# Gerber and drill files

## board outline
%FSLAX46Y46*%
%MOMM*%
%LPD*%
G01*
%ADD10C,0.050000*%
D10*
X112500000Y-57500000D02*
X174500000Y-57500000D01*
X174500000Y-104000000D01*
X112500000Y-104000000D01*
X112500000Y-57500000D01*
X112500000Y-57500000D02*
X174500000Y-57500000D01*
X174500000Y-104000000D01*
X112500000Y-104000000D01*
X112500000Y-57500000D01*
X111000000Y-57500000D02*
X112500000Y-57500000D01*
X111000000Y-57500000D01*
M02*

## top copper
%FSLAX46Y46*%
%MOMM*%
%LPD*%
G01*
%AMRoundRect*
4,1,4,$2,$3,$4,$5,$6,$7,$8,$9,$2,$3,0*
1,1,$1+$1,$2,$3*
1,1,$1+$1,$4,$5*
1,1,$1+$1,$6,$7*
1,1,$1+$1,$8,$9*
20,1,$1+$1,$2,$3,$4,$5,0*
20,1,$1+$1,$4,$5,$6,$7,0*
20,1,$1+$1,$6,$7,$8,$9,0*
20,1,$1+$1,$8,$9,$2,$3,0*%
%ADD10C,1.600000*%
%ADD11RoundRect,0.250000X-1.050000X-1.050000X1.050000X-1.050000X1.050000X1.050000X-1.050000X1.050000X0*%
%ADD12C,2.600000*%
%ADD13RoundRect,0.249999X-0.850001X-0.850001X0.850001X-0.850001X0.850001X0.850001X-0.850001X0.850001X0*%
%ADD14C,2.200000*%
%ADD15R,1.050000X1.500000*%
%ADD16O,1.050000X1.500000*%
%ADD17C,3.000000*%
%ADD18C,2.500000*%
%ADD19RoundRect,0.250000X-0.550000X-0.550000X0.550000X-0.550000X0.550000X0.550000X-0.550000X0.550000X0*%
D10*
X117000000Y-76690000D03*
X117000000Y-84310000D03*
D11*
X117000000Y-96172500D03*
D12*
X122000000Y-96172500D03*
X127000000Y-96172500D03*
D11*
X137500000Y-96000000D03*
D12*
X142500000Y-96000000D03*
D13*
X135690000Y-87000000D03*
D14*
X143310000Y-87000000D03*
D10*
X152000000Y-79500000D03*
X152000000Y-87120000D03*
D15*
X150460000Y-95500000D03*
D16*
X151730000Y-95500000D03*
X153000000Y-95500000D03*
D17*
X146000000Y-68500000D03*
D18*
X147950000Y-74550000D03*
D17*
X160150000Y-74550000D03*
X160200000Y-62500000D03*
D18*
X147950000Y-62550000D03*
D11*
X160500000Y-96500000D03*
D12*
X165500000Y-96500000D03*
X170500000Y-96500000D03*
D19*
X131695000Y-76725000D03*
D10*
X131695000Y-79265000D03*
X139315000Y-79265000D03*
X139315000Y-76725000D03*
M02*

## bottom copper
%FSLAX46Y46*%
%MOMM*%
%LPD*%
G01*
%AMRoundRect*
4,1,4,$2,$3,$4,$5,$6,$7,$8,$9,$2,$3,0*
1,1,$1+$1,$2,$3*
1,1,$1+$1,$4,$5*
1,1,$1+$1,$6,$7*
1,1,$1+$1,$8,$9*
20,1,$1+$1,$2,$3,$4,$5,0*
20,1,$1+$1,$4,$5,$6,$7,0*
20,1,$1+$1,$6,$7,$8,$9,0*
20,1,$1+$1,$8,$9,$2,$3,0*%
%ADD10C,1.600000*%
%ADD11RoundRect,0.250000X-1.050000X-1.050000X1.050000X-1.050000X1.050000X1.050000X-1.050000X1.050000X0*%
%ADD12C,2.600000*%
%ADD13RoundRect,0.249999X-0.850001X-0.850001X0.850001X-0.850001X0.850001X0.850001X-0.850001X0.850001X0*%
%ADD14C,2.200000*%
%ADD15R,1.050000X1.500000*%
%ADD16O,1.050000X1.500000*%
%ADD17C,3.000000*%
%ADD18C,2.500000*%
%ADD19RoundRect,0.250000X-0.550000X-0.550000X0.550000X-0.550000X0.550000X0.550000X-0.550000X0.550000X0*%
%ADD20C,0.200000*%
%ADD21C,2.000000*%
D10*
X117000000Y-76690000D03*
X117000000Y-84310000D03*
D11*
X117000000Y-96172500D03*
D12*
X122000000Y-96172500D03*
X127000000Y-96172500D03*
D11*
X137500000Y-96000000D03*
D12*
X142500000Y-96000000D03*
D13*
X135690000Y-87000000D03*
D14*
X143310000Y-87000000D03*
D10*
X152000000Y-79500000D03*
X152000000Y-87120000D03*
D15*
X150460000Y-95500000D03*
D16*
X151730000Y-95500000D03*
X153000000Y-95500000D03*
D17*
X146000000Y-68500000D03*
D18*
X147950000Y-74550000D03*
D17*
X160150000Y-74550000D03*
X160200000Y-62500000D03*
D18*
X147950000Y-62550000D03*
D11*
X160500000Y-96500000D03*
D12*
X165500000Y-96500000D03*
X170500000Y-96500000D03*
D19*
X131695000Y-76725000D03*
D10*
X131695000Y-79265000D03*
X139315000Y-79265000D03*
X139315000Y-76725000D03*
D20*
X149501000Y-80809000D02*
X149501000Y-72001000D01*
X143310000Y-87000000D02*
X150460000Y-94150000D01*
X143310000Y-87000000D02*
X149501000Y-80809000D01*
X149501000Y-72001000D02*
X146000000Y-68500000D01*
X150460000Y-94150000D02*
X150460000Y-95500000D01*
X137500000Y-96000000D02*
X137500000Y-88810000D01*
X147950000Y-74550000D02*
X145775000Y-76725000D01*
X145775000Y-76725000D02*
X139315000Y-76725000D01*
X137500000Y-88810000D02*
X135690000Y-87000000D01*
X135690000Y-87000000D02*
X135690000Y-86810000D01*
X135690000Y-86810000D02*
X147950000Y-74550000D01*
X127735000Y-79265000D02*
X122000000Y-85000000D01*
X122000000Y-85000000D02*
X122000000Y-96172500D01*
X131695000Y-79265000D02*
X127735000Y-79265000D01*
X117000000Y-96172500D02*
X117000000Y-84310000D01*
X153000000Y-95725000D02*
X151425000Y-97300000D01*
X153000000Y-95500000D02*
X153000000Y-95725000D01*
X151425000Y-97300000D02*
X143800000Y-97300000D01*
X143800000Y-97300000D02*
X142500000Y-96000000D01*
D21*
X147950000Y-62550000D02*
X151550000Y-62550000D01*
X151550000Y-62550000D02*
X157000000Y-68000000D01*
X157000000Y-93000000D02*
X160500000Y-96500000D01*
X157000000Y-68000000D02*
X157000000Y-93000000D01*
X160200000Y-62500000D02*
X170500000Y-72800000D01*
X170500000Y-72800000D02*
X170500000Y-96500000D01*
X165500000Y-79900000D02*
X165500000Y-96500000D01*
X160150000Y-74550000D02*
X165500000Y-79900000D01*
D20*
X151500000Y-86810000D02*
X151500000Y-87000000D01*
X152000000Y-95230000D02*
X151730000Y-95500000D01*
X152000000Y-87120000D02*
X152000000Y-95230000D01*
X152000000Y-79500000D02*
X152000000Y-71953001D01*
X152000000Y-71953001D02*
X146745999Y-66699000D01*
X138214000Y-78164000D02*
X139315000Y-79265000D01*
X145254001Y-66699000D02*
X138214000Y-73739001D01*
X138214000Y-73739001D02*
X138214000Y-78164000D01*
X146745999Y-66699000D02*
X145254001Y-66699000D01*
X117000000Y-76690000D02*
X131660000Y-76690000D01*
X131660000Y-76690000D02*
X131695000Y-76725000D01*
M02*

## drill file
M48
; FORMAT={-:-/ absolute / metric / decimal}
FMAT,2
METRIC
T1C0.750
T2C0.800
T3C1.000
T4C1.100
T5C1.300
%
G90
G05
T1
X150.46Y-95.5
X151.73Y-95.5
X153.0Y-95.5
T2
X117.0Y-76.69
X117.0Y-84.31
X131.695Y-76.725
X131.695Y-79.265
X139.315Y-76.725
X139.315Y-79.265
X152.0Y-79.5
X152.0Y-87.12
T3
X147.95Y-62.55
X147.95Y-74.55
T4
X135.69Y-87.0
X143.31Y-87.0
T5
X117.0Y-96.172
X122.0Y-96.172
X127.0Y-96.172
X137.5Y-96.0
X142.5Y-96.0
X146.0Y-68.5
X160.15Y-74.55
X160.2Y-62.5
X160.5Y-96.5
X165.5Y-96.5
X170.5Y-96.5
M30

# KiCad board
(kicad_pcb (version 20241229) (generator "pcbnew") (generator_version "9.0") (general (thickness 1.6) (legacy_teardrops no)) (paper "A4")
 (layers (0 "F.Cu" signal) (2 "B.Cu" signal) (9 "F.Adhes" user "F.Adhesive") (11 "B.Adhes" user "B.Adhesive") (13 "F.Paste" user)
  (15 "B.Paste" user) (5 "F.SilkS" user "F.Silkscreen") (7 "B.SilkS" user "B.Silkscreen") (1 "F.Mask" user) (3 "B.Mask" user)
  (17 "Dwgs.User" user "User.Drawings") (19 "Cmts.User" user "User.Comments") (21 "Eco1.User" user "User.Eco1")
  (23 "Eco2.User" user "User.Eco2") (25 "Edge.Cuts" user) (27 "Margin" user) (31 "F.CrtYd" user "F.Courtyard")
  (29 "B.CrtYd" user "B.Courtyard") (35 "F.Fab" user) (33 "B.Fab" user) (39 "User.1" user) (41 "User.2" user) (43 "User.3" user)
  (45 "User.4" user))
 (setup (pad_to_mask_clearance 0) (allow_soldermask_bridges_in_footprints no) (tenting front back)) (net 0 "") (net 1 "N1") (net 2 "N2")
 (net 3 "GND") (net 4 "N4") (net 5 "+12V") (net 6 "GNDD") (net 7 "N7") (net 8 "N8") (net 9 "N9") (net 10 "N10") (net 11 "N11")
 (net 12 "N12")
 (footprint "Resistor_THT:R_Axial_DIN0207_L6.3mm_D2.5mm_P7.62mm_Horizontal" (layer "F.Cu") (at 117 76.69 -90)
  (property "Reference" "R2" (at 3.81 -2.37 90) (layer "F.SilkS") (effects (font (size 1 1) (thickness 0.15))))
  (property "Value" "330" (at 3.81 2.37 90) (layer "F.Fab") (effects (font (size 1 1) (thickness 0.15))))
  (pad "1" thru_hole circle (at 0 0 270) (size 1.6 1.6) (drill 0.8) (layers "*.Cu" "*.Mask") (remove_unused_layers no) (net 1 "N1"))
  (pad "2" thru_hole circle (at 7.62 0 270) (size 1.6 1.6) (drill 0.8) (layers "*.Cu" "*.Mask") (remove_unused_layers no) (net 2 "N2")))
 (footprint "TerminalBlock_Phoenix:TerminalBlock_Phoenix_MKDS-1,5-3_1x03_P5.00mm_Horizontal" (layer "F.Cu") (at 117 96.1725)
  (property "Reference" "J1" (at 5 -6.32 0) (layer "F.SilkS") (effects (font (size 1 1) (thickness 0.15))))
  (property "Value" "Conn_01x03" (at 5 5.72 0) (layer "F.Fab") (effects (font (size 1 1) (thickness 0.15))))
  (pad "1" thru_hole roundrect (at 0 0) (size 2.6 2.6) (drill 1.3) (layers "*.Cu" "*.Mask") (remove_unused_layers no)
   (roundrect_rratio 0.096154) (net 2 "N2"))
  (pad "2" thru_hole circle (at 5 0) (size 2.6 2.6) (drill 1.3) (layers "*.Cu" "*.Mask") (remove_unused_layers no) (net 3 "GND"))
  (pad "3" thru_hole circle (at 10 0) (size 2.6 2.6) (drill 1.3) (layers "*.Cu" "*.Mask") (remove_unused_layers no) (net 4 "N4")))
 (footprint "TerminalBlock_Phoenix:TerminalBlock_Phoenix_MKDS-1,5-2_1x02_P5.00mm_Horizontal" (layer "F.Cu") (at 137.5 96)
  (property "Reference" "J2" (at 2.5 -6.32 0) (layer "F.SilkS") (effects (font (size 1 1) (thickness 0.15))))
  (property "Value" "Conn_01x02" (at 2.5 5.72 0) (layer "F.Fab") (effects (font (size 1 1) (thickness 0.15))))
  (pad "1" thru_hole roundrect (at 0 0) (size 2.6 2.6) (drill 1.3) (layers "*.Cu" "*.Mask") (remove_unused_layers no)
   (roundrect_rratio 0.096154) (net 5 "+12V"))
  (pad "2" thru_hole circle (at 5 0) (size 2.6 2.6) (drill 1.3) (layers "*.Cu" "*.Mask") (remove_unused_layers no) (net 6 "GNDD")))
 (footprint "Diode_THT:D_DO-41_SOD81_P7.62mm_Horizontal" (layer "F.Cu") (at 135.69 87)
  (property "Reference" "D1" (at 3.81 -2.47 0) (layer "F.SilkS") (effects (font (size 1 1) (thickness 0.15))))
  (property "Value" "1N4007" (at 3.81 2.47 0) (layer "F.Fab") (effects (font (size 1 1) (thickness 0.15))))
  (pad "1" thru_hole roundrect (at 0 0) (size 2.2 2.2) (drill 1.1) (layers "*.Cu" "*.Mask") (remove_unused_layers no)
   (roundrect_rratio 0.113636) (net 5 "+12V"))
  (pad "2" thru_hole circle (at 7.62 0) (size 2.2 2.2) (drill 1.1) (layers "*.Cu" "*.Mask") (remove_unused_layers no) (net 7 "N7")))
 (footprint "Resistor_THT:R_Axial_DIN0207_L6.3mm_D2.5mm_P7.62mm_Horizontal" (layer "F.Cu") (at 152 79.5 -90)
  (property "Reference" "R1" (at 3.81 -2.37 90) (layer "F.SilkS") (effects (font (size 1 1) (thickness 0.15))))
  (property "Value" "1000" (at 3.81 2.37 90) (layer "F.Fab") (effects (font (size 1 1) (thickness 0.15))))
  (pad "1" thru_hole circle (at 0 0 270) (size 1.6 1.6) (drill 0.8) (layers "*.Cu" "*.Mask") (remove_unused_layers no) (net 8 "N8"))
  (pad "2" thru_hole circle (at 7.62 0 270) (size 1.6 1.6) (drill 0.8) (layers "*.Cu" "*.Mask") (remove_unused_layers no) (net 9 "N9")))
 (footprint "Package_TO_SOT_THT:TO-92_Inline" (layer "F.Cu") (at 150.46 95.5)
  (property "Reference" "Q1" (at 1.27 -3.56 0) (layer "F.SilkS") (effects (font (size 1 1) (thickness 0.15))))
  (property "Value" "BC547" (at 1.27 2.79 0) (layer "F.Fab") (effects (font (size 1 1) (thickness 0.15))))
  (pad "1" thru_hole rect (at 0 0) (size 1.05 1.5) (drill 0.75) (layers "*.Cu" "*.Mask") (remove_unused_layers no) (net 7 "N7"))
  (pad "2" thru_hole oval (at 1.27 0) (size 1.05 1.5) (drill 0.75) (layers "*.Cu" "*.Mask") (remove_unused_layers no) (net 9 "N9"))
  (pad "3" thru_hole oval (at 2.54 0) (size 1.05 1.5) (drill 0.75) (layers "*.Cu" "*.Mask") (remove_unused_layers no) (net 6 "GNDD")))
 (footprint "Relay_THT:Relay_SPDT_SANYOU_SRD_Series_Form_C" (layer "F.Cu") (at 146 68.5)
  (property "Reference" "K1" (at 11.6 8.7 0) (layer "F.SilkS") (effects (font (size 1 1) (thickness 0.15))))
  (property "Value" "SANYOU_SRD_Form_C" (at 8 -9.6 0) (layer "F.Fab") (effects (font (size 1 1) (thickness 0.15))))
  (pad "1" thru_hole circle (at 0 0 90) (size 3 3) (drill 1.3) (layers "*.Cu" "*.Mask") (remove_unused_layers no) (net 7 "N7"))
  (pad "2" thru_hole circle (at 1.95 6.05 90) (size 2.5 2.5) (drill 1) (layers "*.Cu" "*.Mask") (remove_unused_layers no) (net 5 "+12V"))
  (pad "3" thru_hole circle (at 14.15 6.05 90) (size 3 3) (drill 1.3) (layers "*.Cu" "*.Mask") (remove_unused_layers no) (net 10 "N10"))
  (pad "4" thru_hole circle (at 14.2 -6 90) (size 3 3) (drill 1.3) (layers "*.Cu" "*.Mask") (remove_unused_layers no) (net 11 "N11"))
  (pad "5" thru_hole circle (at 1.95 -5.95 90) (size 2.5 2.5) (drill 1) (layers "*.Cu" "*.Mask") (remove_unused_layers no) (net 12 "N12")))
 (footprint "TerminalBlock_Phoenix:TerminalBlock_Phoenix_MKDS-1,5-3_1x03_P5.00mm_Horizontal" (layer "F.Cu") (at 160.5 96.5)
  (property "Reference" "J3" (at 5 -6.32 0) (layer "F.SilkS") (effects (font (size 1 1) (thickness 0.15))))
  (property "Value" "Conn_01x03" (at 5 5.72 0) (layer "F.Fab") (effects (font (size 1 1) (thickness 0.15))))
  (pad "1" thru_hole roundrect (at 0 0) (size 2.6 2.6) (drill 1.3) (layers "*.Cu" "*.Mask") (remove_unused_layers no)
   (roundrect_rratio 0.096154) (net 12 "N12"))
  (pad "2" thru_hole circle (at 5 0) (size 2.6 2.6) (drill 1.3) (layers "*.Cu" "*.Mask") (remove_unused_layers no) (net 10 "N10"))
  (pad "3" thru_hole circle (at 10 0) (size 2.6 2.6) (drill 1.3) (layers "*.Cu" "*.Mask") (remove_unused_layers no) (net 11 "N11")))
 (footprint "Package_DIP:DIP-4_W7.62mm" (layer "F.Cu") (at 131.695 76.725)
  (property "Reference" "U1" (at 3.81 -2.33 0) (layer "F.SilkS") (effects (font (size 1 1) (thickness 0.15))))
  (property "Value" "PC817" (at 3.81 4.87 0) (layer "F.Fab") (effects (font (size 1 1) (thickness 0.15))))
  (pad "1" thru_hole roundrect (at 0 0) (size 1.6 1.6) (drill 0.8) (layers "*.Cu" "*.Mask") (remove_unused_layers no)
   (roundrect_rratio 0.15625) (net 1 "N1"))
  (pad "2" thru_hole circle (at 0 2.54) (size 1.6 1.6) (drill 0.8) (layers "*.Cu" "*.Mask") (remove_unused_layers no) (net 3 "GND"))
  (pad "3" thru_hole circle (at 7.62 2.54) (size 1.6 1.6) (drill 0.8) (layers "*.Cu" "*.Mask") (remove_unused_layers no) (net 8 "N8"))
  (pad "4" thru_hole circle (at 7.62 0) (size 1.6 1.6) (drill 0.8) (layers "*.Cu" "*.Mask") (remove_unused_layers no) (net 5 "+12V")))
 (gr_rect (start 112.5 57.5) (end 174.5 104) (stroke (width 0.05) (type default)) (fill no) (layer "Edge.Cuts"))
 (gr_rect (start 112.5 57.5) (end 174.5 104) (stroke (width 0.05) (type default)) (fill no) (layer "Edge.Cuts"))
 (gr_rect (start 111 57.5) (end 112.5 57.5) (stroke (width 0.05) (type default)) (fill no) (layer "Edge.Cuts"))
 (segment (start 149.501 80.809) (end 149.501 72.001) (width 0.2) (layer "B.Cu") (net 7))
 (segment (start 143.31 87) (end 150.46 94.15) (width 0.2) (layer "B.Cu") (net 7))
 (segment (start 143.31 87) (end 149.501 80.809) (width 0.2) (layer "B.Cu") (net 7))
 (segment (start 149.501 72.001) (end 146 68.5) (width 0.2) (layer "B.Cu") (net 7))
 (segment (start 150.46 94.15) (end 150.46 95.5) (width 0.2) (layer "B.Cu") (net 7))
 (segment (start 137.5 96) (end 137.5 88.81) (width 0.2) (layer "B.Cu") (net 5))
 (segment (start 147.95 74.55) (end 145.775 76.725) (width 0.2) (layer "B.Cu") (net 5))
 (segment (start 145.775 76.725) (end 139.315 76.725) (width 0.2) (layer "B.Cu") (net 5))
 (segment (start 137.5 88.81) (end 135.69 87) (width 0.2) (layer "B.Cu") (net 5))
 (segment (start 135.69 87) (end 135.69 86.81) (width 0.2) (layer "B.Cu") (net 5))
 (segment (start 135.69 86.81) (end 147.95 74.55) (width 0.2) (layer "B.Cu") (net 5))
 (segment (start 127.735 79.265) (end 122 85) (width 0.2) (layer "B.Cu") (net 3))
 (segment (start 122 85) (end 122 96.1725) (width 0.2) (layer "B.Cu") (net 3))
 (segment (start 131.695 79.265) (end 127.735 79.265) (width 0.2) (layer "B.Cu") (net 3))
 (segment (start 117 96.1725) (end 117 84.31) (width 0.2) (layer "B.Cu") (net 2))
 (segment (start 153 95.725) (end 151.425 97.3) (width 0.2) (layer "B.Cu") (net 6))
 (segment (start 153 95.5) (end 153 95.725) (width 0.2) (layer "B.Cu") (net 6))
 (segment (start 151.425 97.3) (end 143.8 97.3) (width 0.2) (layer "B.Cu") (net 6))
 (segment (start 143.8 97.3) (end 142.5 96) (width 0.2) (layer "B.Cu") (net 6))
 (segment (start 147.95 62.55) (end 151.55 62.55) (width 2) (layer "B.Cu") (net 12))
 (segment (start 151.55 62.55) (end 157 68) (width 2) (layer "B.Cu") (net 12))
 (segment (start 157 93) (end 160.5 96.5) (width 2) (layer "B.Cu") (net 12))
 (segment (start 157 68) (end 157 93) (width 2) (layer "B.Cu") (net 12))
 (segment (start 160.2 62.5) (end 170.5 72.8) (width 2) (layer "B.Cu") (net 11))
 (segment (start 170.5 72.8) (end 170.5 96.5) (width 2) (layer "B.Cu") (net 11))
 (segment (start 165.5 79.9) (end 165.5 96.5) (width 2) (layer "B.Cu") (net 10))
 (segment (start 160.15 74.55) (end 165.5 79.9) (width 2) (layer "B.Cu") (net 10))
 (segment (start 151.5 86.81) (end 151.5 87) (width 0.2) (layer "B.Cu") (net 9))
 (segment (start 152 95.23) (end 151.73 95.5) (width 0.2) (layer "B.Cu") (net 9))
 (segment (start 152 87.12) (end 152 95.23) (width 0.2) (layer "B.Cu") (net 9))
 (segment (start 152 79.5) (end 152 71.953001) (width 0.2) (layer "B.Cu") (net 8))
 (segment (start 152 71.953001) (end 146.745999 66.699) (width 0.2) (layer "B.Cu") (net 8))
 (segment (start 138.214 78.164) (end 139.315 79.265) (width 0.2) (layer "B.Cu") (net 8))
 (segment (start 145.254001 66.699) (end 138.214 73.739001) (width 0.2) (layer "B.Cu") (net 8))
 (segment (start 138.214 73.739001) (end 138.214 78.164) (width 0.2) (layer "B.Cu") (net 8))
 (segment (start 146.745999 66.699) (end 145.254001 66.699) (width 0.2) (layer "B.Cu") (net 8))
 (segment (start 117 76.69) (end 131.66 76.69) (width 0.2) (layer "B.Cu") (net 1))
 (segment (start 131.66 76.69) (end 131.695 76.725) (width 0.2) (layer "B.Cu") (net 1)))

